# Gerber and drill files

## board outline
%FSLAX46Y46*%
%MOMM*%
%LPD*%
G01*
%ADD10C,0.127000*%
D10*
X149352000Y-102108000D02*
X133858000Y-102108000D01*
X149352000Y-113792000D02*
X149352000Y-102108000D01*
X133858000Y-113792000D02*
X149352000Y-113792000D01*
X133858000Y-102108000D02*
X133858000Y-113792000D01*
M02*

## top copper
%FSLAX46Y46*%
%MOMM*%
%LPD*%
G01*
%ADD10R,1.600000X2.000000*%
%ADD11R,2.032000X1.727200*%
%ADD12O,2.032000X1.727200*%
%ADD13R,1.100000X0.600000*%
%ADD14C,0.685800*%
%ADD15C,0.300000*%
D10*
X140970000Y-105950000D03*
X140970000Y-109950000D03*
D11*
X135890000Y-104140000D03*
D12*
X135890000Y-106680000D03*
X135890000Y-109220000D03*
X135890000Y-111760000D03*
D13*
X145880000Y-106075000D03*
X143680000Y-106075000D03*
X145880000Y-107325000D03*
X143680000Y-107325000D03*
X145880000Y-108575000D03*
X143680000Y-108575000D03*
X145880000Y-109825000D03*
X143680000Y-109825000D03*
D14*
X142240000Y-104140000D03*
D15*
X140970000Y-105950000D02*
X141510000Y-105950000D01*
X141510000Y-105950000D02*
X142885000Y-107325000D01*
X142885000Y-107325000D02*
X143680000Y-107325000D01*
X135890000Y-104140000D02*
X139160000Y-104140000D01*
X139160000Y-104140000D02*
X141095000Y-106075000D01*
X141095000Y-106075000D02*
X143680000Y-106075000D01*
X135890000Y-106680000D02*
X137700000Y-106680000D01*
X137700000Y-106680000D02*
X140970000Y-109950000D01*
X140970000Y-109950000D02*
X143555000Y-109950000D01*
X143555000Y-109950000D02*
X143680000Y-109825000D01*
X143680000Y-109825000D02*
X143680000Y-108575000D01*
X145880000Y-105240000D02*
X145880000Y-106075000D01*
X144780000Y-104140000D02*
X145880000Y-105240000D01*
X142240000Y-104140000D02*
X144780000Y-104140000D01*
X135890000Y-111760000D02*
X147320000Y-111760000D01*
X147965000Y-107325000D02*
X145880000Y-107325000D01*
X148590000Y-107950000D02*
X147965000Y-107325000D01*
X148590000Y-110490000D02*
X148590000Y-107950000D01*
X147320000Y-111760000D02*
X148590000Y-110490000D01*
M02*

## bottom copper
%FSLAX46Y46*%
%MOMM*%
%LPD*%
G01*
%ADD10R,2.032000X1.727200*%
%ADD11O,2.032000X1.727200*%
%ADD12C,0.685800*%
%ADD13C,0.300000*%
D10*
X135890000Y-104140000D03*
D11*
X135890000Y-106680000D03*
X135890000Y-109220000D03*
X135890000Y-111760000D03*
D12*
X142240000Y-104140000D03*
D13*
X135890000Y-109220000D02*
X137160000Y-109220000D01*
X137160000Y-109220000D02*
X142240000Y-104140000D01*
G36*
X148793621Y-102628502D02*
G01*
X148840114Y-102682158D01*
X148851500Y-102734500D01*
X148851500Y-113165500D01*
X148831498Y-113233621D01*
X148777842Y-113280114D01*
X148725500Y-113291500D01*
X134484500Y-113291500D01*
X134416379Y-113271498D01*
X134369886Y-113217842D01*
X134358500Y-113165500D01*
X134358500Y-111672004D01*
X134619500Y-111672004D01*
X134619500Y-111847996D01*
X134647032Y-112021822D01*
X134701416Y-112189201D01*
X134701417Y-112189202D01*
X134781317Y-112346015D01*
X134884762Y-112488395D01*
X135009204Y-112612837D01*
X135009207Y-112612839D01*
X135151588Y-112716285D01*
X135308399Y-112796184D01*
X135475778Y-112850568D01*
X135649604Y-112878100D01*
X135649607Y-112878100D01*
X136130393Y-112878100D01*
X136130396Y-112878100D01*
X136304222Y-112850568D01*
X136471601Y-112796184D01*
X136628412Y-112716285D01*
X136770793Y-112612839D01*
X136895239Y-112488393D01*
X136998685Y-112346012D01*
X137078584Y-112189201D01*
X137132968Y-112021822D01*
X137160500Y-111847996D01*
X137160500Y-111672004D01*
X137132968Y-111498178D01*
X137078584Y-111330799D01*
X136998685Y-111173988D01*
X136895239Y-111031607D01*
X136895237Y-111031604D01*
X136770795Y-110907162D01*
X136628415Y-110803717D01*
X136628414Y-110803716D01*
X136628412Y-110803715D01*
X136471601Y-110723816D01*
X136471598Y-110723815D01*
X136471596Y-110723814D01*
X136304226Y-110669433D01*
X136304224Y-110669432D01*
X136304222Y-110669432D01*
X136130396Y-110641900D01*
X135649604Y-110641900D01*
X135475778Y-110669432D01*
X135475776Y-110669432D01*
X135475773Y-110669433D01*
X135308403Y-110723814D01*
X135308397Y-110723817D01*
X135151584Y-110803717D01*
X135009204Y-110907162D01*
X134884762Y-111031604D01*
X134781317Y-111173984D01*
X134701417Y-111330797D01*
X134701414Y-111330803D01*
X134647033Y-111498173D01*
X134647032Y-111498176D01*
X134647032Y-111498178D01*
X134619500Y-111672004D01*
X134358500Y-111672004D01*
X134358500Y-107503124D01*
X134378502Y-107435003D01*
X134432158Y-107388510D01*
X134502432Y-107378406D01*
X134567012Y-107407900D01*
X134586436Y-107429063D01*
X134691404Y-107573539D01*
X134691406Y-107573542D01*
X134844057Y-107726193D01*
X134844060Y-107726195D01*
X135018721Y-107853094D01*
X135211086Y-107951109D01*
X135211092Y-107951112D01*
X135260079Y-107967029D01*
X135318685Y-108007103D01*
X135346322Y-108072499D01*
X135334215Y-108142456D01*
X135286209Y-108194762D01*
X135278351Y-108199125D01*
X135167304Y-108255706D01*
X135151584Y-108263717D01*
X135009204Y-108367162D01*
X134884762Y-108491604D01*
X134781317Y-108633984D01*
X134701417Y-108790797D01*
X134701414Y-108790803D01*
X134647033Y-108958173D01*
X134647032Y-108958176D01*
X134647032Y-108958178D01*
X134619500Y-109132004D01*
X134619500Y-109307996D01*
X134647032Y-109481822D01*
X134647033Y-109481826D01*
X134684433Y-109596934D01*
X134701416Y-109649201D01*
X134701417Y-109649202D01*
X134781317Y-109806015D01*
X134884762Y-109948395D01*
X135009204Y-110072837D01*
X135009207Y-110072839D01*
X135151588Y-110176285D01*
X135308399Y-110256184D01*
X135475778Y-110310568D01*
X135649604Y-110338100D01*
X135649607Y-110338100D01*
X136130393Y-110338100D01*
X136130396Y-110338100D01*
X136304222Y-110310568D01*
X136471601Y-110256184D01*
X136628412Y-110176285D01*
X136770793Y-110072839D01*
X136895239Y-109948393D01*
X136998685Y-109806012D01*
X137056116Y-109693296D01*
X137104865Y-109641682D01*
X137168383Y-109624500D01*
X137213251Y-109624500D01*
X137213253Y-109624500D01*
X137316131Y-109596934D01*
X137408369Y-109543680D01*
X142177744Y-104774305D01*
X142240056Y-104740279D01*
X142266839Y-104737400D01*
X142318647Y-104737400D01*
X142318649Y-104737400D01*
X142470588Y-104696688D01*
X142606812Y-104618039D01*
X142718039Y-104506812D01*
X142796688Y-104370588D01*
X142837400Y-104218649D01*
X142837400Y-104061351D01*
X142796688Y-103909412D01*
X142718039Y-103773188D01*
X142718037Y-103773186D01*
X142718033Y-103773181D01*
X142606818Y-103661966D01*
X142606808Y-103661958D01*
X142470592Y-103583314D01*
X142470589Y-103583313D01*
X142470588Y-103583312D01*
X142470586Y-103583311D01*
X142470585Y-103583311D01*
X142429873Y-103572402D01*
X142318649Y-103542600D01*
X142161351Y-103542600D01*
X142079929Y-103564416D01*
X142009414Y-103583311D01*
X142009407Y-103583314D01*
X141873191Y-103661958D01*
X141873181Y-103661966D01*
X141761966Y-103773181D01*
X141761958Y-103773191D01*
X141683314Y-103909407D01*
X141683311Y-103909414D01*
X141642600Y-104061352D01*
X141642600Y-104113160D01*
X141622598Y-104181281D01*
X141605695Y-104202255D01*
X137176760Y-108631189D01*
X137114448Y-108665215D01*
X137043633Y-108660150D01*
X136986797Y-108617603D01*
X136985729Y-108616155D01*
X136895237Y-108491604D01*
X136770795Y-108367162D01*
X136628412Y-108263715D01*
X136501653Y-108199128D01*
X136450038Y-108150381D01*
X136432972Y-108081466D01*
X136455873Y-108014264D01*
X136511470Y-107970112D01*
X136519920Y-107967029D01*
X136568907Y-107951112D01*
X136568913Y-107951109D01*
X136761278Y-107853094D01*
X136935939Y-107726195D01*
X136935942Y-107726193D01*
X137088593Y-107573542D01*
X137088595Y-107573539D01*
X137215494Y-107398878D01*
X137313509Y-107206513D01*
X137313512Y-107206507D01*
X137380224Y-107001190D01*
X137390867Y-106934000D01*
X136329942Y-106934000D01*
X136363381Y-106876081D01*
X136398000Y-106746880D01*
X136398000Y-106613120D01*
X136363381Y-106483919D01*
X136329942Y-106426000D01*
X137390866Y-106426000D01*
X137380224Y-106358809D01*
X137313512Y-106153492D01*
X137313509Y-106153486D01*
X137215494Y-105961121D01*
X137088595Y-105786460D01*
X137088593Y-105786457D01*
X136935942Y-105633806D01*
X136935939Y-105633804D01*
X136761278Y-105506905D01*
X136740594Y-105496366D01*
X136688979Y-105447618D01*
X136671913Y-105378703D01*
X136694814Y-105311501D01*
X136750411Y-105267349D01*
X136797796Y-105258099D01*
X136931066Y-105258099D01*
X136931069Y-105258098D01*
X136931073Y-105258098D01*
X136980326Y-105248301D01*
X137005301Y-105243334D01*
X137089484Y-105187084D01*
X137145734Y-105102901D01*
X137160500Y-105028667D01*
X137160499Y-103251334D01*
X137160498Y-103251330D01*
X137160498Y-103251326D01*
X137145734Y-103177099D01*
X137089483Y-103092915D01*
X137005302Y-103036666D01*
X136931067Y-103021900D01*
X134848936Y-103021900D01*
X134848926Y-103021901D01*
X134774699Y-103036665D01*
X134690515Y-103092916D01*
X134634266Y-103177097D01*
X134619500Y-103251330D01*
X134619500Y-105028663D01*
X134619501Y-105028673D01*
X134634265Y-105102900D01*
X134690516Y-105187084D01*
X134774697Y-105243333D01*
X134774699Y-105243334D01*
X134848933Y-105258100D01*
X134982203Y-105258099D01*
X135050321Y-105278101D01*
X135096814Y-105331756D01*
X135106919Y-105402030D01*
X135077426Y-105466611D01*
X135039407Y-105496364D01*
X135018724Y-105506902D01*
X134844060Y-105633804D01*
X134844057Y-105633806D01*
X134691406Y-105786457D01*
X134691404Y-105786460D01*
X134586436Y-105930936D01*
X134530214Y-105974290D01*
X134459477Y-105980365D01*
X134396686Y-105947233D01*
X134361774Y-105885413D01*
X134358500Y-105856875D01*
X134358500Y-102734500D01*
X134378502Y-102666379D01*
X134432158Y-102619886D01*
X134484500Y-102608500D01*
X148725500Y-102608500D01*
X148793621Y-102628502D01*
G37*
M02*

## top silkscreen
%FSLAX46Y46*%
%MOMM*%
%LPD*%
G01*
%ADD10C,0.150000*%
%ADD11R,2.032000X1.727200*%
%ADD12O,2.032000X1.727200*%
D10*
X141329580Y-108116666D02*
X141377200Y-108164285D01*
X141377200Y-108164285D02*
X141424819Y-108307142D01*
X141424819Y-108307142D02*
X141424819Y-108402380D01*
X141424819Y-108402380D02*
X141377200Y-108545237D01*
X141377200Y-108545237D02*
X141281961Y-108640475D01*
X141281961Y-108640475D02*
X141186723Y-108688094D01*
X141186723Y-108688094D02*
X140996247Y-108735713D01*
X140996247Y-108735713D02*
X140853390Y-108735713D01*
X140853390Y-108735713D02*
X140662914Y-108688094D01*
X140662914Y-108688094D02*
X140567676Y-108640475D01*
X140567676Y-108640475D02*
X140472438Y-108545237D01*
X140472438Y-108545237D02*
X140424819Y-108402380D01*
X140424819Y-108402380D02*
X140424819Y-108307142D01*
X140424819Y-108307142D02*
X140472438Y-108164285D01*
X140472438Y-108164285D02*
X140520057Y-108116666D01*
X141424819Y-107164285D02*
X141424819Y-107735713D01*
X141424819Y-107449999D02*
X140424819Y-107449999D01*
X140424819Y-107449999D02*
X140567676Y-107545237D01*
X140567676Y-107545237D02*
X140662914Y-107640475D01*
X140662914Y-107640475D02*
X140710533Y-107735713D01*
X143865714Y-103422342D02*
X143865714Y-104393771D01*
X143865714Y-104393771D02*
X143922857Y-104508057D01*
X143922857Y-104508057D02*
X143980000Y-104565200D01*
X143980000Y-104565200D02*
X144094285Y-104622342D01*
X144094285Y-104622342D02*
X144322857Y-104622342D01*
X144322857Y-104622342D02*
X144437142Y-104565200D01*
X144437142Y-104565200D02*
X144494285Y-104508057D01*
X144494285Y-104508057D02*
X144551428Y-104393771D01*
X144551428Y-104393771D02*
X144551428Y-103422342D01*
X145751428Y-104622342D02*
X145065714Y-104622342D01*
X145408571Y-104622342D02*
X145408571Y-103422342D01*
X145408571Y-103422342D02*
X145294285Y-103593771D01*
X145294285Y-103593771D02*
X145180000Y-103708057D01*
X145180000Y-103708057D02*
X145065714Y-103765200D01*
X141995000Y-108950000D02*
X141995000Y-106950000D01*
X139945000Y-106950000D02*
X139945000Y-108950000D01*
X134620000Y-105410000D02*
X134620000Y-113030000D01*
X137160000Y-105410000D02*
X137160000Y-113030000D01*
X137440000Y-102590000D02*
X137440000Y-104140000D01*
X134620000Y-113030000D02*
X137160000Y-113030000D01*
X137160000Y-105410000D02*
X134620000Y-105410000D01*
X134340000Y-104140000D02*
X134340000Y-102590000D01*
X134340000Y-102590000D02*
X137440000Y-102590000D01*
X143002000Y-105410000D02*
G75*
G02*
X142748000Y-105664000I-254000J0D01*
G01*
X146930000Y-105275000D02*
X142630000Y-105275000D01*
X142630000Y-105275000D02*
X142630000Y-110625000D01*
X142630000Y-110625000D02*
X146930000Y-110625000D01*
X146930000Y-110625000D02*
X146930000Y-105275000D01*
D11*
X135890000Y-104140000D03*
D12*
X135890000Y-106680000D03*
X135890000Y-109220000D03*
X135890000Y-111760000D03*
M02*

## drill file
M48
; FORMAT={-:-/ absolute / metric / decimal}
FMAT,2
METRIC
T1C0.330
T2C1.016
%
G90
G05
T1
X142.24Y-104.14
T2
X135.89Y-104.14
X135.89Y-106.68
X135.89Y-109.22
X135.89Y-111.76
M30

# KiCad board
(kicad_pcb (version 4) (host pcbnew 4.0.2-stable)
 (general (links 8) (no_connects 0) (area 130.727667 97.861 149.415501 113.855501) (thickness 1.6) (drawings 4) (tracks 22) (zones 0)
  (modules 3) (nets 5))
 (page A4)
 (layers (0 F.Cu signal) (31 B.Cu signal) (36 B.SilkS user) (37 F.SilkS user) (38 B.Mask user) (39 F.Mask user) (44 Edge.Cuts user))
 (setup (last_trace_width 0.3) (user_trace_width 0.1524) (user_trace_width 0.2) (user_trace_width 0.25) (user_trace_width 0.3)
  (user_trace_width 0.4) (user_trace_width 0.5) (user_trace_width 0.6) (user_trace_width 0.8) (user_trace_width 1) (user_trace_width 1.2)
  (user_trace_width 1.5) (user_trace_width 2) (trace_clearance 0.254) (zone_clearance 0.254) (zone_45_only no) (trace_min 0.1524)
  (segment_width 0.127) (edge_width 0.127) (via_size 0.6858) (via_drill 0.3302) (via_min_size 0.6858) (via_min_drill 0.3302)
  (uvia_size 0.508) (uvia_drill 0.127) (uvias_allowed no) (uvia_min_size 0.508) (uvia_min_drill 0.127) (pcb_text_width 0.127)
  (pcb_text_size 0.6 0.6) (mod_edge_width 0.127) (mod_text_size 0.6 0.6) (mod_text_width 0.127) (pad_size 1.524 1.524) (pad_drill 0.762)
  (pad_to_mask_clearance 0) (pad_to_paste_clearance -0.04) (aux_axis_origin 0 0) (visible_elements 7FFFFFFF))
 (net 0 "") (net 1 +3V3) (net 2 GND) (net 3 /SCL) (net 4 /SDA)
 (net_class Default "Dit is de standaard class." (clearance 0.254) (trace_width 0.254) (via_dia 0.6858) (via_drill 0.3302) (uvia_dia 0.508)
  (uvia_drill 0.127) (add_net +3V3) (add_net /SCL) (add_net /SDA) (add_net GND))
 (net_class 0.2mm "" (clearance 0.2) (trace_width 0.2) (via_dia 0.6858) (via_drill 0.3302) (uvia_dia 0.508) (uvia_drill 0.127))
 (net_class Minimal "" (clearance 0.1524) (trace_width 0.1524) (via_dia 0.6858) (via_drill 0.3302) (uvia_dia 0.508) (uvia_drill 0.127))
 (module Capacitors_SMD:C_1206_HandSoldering (layer F.Cu) (at 140.97 107.95 270)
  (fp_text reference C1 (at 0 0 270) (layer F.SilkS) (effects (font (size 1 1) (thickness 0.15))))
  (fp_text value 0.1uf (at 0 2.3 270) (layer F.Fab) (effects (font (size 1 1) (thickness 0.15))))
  (fp_line (start 1 -1.025) (end -1 -1.025) (layer F.SilkS) (width 0.15))
  (fp_line (start -1 1.025) (end 1 1.025) (layer F.SilkS) (width 0.15))
  (pad 1 smd rect (at -2 0 270) (size 2 1.6) (layers F.Cu F.Mask) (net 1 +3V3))
  (pad 2 smd rect (at 2 0 270) (size 2 1.6) (layers F.Cu F.Mask) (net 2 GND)))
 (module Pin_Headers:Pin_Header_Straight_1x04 (layer F.Cu) (at 135.89 104.14)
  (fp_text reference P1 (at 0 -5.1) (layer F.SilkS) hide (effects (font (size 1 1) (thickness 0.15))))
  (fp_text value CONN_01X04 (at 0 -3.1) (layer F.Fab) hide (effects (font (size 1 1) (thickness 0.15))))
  (fp_line (start -1.27 1.27) (end -1.27 8.89) (layer F.SilkS) (width 0.15))
  (fp_line (start 1.27 1.27) (end 1.27 8.89) (layer F.SilkS) (width 0.15))
  (fp_line (start 1.55 -1.55) (end 1.55 0) (layer F.SilkS) (width 0.15))
  (fp_line (start -1.27 8.89) (end 1.27 8.89) (layer F.SilkS) (width 0.15))
  (fp_line (start 1.27 1.27) (end -1.27 1.27) (layer F.SilkS) (width 0.15))
  (fp_line (start -1.55 0) (end -1.55 -1.55) (layer F.SilkS) (width 0.15))
  (fp_line (start -1.55 -1.55) (end 1.55 -1.55) (layer F.SilkS) (width 0.15))
  (pad 1 thru_hole rect (at 0 0) (size 2.032 1.7272) (drill 1.016) (layers *.Cu *.Mask F.SilkS) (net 1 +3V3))
  (pad 2 thru_hole oval (at 0 2.54) (size 2.032 1.7272) (drill 1.016) (layers *.Cu *.Mask F.SilkS) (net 2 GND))
  (pad 3 thru_hole oval (at 0 5.08) (size 2.032 1.7272) (drill 1.016) (layers *.Cu *.Mask F.SilkS) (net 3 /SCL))
  (pad 4 thru_hole oval (at 0 7.62) (size 2.032 1.7272) (drill 1.016) (layers *.Cu *.Mask F.SilkS) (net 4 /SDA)))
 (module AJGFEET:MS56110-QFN (layer F.Cu) (at 144.78 107.95 270)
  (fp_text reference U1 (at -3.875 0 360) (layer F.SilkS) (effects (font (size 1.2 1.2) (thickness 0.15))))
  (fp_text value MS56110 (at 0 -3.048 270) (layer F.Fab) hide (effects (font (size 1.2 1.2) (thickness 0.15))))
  (fp_arc (start -2.54 2.032) (end -2.54 1.778) (angle 90) (layer F.SilkS) (width 0.15))
  (fp_line (start -2.675 -2.15) (end -2.675 2.15) (layer F.SilkS) (width 0.15))
  (fp_line (start -2.675 2.15) (end 2.675 2.15) (layer F.SilkS) (width 0.15))
  (fp_line (start 2.675 2.15) (end 2.675 -2.15) (layer F.SilkS) (width 0.15))
  (fp_line (start 2.675 -2.15) (end -2.675 -2.15) (layer F.SilkS) (width 0.15))
  (pad 8 smd rect (at -1.875 -1.1 270) (size 0.6 1.1) (layers F.Cu F.Mask) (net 3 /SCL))
  (pad 1 smd rect (at -1.875 1.1 270) (size 0.6 1.1) (layers F.Cu F.Mask) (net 1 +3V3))
  (pad 7 smd rect (at -0.625 -1.1 270) (size 0.6 1.1) (layers F.Cu F.Mask) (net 4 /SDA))
  (pad 2 smd rect (at -0.625 1.1 270) (size 0.6 1.1) (layers F.Cu F.Mask) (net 1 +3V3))
  (pad 6 smd rect (at 0.625 -1.1 270) (size 0.6 1.1) (layers F.Cu F.Mask))
  (pad 3 smd rect (at 0.625 1.1 270) (size 0.6 1.1) (layers F.Cu F.Mask) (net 2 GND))
  (pad 5 smd rect (at 1.875 -1.1 270) (size 0.6 1.1) (layers F.Cu F.Mask))
  (pad 4 smd rect (at 1.875 1.1 270) (size 0.6 1.1) (layers F.Cu F.Mask) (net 2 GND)))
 (gr_line (start 149.352 102.108) (end 133.858 102.108) (angle 90) (layer Edge.Cuts) (width 0.127))
 (gr_line (start 149.352 113.792) (end 149.352 102.108) (angle 90) (layer Edge.Cuts) (width 0.127))
 (gr_line (start 133.858 113.792) (end 149.352 113.792) (angle 90) (layer Edge.Cuts) (width 0.127))
 (gr_line (start 133.858 102.108) (end 133.858 113.792) (angle 90) (layer Edge.Cuts) (width 0.127))
 (segment (start 140.97 105.95) (end 141.51 105.95) (width 0.3) (layer F.Cu) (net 1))
 (segment (start 141.51 105.95) (end 142.885 107.325) (width 0.3) (layer F.Cu) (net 1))
 (segment (start 142.885 107.325) (end 143.68 107.325) (width 0.3) (layer F.Cu) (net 1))
 (segment (start 135.89 104.14) (end 139.16 104.14) (width 0.3) (layer F.Cu) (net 1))
 (segment (start 139.16 104.14) (end 141.095 106.075) (width 0.3) (layer F.Cu) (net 1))
 (segment (start 141.095 106.075) (end 143.68 106.075) (width 0.3) (layer F.Cu) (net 1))
 (segment (start 135.89 106.68) (end 137.7 106.68) (width 0.3) (layer F.Cu) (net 2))
 (segment (start 137.7 106.68) (end 140.97 109.95) (width 0.3) (layer F.Cu) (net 2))
 (segment (start 140.97 109.95) (end 143.555 109.95) (width 0.3) (layer F.Cu) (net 2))
 (segment (start 143.555 109.95) (end 143.68 109.825) (width 0.3) (layer F.Cu) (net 2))
 (segment (start 143.68 109.825) (end 143.68 108.575) (width 0.3) (layer F.Cu) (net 2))
 (segment (start 135.89 109.22) (end 137.16 109.22) (width 0.3) (layer B.Cu) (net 3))
 (segment (start 145.88 105.24) (end 145.88 106.075) (width 0.3) (layer F.Cu) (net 3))
 (segment (start 144.78 104.14) (end 145.88 105.24) (width 0.3) (layer F.Cu) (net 3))
 (segment (start 142.24 104.14) (end 144.78 104.14) (width 0.3) (layer F.Cu) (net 3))
 (via (at 142.24 104.14) (size 0.6858) (drill 0.3302) (layers F.Cu B.Cu) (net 3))
 (segment (start 137.16 109.22) (end 142.24 104.14) (width 0.3) (layer B.Cu) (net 3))
 (segment (start 135.89 111.76) (end 147.32 111.76) (width 0.3) (layer F.Cu) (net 4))
 (segment (start 147.965 107.325) (end 145.88 107.325) (width 0.3) (layer F.Cu) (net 4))
 (segment (start 148.59 107.95) (end 147.965 107.325) (width 0.3) (layer F.Cu) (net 4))
 (segment (start 148.59 110.49) (end 148.59 107.95) (width 0.3) (layer F.Cu) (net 4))
 (segment (start 147.32 111.76) (end 148.59 110.49) (width 0.3) (layer F.Cu) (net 4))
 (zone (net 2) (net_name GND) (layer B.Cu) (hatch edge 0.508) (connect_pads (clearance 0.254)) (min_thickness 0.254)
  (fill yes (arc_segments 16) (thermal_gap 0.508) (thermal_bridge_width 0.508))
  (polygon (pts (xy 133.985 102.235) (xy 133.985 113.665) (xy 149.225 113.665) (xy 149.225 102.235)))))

